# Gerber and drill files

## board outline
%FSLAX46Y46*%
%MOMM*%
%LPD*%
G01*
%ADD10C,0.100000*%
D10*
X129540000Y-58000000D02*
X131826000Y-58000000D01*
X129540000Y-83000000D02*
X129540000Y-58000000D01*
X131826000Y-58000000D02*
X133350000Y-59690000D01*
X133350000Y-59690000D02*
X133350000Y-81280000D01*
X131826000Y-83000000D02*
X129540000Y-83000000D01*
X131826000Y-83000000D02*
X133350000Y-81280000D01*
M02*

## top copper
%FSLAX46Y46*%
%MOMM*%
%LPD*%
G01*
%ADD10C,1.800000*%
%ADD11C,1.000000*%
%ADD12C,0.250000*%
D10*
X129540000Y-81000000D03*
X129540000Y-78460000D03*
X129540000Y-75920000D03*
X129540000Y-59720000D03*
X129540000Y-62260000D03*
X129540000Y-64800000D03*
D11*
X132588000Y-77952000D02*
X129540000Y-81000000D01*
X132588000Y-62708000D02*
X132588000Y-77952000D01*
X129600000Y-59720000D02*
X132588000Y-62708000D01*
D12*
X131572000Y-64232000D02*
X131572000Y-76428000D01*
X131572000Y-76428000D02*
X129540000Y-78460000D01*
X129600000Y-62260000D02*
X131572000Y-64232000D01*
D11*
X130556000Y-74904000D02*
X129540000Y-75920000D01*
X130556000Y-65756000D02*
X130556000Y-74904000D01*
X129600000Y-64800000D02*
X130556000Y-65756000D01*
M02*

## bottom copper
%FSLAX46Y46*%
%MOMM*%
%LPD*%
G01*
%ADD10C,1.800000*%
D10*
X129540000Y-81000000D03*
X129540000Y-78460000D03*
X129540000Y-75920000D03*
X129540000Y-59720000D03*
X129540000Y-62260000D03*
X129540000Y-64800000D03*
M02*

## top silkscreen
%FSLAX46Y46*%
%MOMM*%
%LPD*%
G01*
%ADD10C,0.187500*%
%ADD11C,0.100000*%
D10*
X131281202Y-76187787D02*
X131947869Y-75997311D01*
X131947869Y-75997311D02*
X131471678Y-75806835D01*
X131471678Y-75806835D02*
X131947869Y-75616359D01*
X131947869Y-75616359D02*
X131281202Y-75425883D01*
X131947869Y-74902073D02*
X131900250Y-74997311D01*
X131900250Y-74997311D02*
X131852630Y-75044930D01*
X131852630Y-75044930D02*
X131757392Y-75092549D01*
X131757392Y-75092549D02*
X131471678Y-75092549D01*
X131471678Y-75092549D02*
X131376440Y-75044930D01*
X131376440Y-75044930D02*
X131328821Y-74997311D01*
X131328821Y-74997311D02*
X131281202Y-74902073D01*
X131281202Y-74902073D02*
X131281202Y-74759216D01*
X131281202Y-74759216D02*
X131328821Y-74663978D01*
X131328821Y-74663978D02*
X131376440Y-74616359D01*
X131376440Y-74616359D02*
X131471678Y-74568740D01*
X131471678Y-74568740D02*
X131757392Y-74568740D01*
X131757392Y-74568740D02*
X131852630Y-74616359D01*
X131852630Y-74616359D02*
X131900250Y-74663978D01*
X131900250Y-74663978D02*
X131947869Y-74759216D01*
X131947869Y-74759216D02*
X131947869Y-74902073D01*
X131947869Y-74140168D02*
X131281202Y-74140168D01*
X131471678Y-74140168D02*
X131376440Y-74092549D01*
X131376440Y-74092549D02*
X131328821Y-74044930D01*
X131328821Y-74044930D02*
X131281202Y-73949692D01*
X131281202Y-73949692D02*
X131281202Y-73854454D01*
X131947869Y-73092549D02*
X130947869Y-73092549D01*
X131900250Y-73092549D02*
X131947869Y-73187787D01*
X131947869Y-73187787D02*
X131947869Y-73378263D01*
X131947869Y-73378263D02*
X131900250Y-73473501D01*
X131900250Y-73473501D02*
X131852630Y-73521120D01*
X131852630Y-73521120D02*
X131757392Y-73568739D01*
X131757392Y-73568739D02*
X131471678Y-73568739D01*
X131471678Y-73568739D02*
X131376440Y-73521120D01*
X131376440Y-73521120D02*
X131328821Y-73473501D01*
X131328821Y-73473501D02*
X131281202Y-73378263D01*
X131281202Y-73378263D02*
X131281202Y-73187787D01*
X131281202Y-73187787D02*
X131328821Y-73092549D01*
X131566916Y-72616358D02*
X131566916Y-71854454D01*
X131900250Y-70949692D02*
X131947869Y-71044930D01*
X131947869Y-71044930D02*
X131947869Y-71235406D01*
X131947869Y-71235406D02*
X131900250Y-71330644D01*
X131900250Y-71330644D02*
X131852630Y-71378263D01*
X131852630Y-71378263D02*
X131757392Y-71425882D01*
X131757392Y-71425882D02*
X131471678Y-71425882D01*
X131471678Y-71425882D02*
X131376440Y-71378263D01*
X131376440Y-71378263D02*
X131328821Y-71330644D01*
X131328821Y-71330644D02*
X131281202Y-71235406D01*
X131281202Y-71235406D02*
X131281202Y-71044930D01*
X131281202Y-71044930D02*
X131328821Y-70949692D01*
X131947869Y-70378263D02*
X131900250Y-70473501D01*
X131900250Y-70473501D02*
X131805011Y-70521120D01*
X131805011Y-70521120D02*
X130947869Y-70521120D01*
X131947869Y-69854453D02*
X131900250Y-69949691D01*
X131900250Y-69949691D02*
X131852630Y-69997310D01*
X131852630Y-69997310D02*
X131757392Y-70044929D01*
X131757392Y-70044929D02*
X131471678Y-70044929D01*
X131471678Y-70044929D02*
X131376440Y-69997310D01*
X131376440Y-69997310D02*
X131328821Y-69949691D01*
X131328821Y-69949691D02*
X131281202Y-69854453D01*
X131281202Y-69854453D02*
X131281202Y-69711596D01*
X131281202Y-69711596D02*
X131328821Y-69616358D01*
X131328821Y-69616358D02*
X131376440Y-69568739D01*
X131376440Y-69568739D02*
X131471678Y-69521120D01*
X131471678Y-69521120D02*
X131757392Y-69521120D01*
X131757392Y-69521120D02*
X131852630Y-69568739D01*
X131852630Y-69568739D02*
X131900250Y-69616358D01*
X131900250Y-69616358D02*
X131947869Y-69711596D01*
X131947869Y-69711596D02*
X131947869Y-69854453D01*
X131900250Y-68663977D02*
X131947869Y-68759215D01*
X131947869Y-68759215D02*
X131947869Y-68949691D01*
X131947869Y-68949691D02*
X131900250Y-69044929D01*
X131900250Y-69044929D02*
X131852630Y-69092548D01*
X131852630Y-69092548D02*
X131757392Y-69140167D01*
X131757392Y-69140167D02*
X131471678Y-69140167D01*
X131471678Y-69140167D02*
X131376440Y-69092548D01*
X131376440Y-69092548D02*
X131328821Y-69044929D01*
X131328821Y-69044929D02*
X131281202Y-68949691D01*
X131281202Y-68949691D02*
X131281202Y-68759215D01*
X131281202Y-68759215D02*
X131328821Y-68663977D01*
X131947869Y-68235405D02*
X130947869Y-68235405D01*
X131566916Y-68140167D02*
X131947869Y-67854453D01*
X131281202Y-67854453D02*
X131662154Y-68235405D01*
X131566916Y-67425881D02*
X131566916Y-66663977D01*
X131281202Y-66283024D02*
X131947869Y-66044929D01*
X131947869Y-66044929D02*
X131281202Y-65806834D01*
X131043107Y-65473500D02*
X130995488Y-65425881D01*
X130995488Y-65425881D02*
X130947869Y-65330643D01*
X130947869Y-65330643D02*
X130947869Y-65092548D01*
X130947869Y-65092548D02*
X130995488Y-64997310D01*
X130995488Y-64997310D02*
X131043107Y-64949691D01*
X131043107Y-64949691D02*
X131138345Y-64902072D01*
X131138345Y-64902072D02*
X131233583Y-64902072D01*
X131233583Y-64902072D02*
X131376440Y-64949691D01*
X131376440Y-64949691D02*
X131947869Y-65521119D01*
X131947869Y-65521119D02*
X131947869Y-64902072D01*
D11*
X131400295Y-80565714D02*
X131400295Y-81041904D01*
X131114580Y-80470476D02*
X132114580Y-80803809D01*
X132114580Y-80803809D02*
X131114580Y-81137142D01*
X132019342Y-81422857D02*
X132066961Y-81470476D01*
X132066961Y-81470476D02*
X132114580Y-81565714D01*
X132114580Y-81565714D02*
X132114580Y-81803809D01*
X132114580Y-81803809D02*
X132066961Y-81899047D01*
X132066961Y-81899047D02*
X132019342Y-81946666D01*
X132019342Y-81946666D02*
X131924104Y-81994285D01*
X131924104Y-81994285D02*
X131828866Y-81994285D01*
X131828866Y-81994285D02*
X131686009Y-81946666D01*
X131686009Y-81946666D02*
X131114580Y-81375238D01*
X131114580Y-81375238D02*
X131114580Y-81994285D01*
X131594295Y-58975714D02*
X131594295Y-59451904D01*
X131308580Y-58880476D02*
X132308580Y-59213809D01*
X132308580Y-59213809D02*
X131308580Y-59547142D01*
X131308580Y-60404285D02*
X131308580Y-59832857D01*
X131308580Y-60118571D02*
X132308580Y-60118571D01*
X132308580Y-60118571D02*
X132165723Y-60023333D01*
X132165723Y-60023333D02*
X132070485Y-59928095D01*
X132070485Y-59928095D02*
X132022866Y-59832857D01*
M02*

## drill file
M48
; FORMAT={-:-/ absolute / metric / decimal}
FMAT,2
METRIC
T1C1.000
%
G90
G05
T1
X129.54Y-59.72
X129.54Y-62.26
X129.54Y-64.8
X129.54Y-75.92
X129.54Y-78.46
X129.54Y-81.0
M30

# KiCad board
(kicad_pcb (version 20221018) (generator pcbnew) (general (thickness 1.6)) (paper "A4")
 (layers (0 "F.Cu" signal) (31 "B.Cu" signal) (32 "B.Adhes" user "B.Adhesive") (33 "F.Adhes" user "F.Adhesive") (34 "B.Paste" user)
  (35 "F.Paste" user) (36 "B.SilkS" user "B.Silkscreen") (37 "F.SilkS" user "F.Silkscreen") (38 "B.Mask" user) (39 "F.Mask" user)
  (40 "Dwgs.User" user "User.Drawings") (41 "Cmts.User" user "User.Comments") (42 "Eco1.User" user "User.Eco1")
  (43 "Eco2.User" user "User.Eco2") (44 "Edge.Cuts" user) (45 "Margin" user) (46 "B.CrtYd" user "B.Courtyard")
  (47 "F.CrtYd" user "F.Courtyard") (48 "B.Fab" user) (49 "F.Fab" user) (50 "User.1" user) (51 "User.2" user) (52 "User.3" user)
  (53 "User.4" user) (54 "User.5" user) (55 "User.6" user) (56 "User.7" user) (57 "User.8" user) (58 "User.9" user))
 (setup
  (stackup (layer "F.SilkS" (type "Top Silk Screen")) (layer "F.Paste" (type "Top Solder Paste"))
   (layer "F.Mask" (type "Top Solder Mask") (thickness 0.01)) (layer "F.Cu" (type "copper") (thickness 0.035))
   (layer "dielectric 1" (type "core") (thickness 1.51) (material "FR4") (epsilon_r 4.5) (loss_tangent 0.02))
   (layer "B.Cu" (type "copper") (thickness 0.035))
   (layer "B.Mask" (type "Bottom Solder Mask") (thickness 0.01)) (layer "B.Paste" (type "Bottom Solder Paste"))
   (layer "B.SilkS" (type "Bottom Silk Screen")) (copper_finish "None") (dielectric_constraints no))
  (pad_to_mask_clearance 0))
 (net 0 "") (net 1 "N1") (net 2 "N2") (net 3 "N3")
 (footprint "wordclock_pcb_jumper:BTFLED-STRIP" (layer "F.Cu") (at 129.54 78.46 180)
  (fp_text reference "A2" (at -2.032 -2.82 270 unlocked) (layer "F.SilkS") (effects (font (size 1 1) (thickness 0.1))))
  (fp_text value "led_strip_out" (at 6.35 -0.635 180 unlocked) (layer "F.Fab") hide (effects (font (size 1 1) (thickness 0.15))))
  (pad "1" thru_hole circle (at 0 -2.54 180) (size 1.8 1.8) (drill 1) (layers "*.Cu" "*.Mask") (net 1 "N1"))
  (pad "2" thru_hole circle (at 0 0 180) (size 1.8 1.8) (drill 1) (layers "*.Cu" "*.Mask") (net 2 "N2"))
  (pad "3" thru_hole circle (at 0 2.54 180) (size 1.8 1.8) (drill 1) (layers "*.Cu" "*.Mask") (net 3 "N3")))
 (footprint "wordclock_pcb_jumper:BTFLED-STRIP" (layer "F.Cu") (at 129.54 62.26)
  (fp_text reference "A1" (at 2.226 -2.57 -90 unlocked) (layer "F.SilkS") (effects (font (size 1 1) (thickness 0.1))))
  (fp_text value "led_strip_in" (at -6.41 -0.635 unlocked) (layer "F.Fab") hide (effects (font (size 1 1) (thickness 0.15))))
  (pad "1" thru_hole circle (at 0 -2.54) (size 1.8 1.8) (drill 1) (layers "*.Cu" "*.Mask") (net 1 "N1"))
  (pad "2" thru_hole circle (at 0 0) (size 1.8 1.8) (drill 1) (layers "*.Cu" "*.Mask") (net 2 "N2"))
  (pad "3" thru_hole circle (at 0 2.54) (size 1.8 1.8) (drill 1) (layers "*.Cu" "*.Mask") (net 3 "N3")))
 (gr_line (start 129.54 58) (end 131.826 58) (stroke (width 0.1) (type default)) (layer "Edge.Cuts"))
 (gr_line (start 129.54 83) (end 129.54 58) (stroke (width 0.1) (type default)) (layer "Edge.Cuts"))
 (gr_line (start 131.826 58) (end 133.35 59.69) (stroke (width 0.1) (type default)) (layer "Edge.Cuts"))
 (gr_line (start 133.35 59.69) (end 133.35 81.28) (stroke (width 0.1) (type default)) (layer "Edge.Cuts"))
 (gr_line (start 131.826 83) (end 129.54 83) (stroke (width 0.1) (type default)) (layer "Edge.Cuts"))
 (gr_line (start 131.826 83) (end 133.35 81.28) (stroke (width 0.1) (type default)) (layer "Edge.Cuts"))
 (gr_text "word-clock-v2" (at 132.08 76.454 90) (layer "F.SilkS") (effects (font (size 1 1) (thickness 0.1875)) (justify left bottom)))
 (segment (start 132.588 77.952) (end 129.54 81) (width 1) (layer "F.Cu") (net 1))
 (segment (start 132.588 62.708) (end 132.588 77.952) (width 1) (layer "F.Cu") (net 1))
 (segment (start 129.6 59.72) (end 132.588 62.708) (width 1) (layer "F.Cu") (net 1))
 (segment (start 131.572 64.232) (end 131.572 76.428) (width 0.25) (layer "F.Cu") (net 2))
 (segment (start 131.572 76.428) (end 129.54 78.46) (width 0.25) (layer "F.Cu") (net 2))
 (segment (start 129.6 62.26) (end 131.572 64.232) (width 0.25) (layer "F.Cu") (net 2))
 (segment (start 130.556 74.904) (end 129.54 75.92) (width 1) (layer "F.Cu") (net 3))
 (segment (start 130.556 65.756) (end 130.556 74.904) (width 1) (layer "F.Cu") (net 3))
 (segment (start 129.6 64.8) (end 130.556 65.756) (width 1) (layer "F.Cu") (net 3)))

